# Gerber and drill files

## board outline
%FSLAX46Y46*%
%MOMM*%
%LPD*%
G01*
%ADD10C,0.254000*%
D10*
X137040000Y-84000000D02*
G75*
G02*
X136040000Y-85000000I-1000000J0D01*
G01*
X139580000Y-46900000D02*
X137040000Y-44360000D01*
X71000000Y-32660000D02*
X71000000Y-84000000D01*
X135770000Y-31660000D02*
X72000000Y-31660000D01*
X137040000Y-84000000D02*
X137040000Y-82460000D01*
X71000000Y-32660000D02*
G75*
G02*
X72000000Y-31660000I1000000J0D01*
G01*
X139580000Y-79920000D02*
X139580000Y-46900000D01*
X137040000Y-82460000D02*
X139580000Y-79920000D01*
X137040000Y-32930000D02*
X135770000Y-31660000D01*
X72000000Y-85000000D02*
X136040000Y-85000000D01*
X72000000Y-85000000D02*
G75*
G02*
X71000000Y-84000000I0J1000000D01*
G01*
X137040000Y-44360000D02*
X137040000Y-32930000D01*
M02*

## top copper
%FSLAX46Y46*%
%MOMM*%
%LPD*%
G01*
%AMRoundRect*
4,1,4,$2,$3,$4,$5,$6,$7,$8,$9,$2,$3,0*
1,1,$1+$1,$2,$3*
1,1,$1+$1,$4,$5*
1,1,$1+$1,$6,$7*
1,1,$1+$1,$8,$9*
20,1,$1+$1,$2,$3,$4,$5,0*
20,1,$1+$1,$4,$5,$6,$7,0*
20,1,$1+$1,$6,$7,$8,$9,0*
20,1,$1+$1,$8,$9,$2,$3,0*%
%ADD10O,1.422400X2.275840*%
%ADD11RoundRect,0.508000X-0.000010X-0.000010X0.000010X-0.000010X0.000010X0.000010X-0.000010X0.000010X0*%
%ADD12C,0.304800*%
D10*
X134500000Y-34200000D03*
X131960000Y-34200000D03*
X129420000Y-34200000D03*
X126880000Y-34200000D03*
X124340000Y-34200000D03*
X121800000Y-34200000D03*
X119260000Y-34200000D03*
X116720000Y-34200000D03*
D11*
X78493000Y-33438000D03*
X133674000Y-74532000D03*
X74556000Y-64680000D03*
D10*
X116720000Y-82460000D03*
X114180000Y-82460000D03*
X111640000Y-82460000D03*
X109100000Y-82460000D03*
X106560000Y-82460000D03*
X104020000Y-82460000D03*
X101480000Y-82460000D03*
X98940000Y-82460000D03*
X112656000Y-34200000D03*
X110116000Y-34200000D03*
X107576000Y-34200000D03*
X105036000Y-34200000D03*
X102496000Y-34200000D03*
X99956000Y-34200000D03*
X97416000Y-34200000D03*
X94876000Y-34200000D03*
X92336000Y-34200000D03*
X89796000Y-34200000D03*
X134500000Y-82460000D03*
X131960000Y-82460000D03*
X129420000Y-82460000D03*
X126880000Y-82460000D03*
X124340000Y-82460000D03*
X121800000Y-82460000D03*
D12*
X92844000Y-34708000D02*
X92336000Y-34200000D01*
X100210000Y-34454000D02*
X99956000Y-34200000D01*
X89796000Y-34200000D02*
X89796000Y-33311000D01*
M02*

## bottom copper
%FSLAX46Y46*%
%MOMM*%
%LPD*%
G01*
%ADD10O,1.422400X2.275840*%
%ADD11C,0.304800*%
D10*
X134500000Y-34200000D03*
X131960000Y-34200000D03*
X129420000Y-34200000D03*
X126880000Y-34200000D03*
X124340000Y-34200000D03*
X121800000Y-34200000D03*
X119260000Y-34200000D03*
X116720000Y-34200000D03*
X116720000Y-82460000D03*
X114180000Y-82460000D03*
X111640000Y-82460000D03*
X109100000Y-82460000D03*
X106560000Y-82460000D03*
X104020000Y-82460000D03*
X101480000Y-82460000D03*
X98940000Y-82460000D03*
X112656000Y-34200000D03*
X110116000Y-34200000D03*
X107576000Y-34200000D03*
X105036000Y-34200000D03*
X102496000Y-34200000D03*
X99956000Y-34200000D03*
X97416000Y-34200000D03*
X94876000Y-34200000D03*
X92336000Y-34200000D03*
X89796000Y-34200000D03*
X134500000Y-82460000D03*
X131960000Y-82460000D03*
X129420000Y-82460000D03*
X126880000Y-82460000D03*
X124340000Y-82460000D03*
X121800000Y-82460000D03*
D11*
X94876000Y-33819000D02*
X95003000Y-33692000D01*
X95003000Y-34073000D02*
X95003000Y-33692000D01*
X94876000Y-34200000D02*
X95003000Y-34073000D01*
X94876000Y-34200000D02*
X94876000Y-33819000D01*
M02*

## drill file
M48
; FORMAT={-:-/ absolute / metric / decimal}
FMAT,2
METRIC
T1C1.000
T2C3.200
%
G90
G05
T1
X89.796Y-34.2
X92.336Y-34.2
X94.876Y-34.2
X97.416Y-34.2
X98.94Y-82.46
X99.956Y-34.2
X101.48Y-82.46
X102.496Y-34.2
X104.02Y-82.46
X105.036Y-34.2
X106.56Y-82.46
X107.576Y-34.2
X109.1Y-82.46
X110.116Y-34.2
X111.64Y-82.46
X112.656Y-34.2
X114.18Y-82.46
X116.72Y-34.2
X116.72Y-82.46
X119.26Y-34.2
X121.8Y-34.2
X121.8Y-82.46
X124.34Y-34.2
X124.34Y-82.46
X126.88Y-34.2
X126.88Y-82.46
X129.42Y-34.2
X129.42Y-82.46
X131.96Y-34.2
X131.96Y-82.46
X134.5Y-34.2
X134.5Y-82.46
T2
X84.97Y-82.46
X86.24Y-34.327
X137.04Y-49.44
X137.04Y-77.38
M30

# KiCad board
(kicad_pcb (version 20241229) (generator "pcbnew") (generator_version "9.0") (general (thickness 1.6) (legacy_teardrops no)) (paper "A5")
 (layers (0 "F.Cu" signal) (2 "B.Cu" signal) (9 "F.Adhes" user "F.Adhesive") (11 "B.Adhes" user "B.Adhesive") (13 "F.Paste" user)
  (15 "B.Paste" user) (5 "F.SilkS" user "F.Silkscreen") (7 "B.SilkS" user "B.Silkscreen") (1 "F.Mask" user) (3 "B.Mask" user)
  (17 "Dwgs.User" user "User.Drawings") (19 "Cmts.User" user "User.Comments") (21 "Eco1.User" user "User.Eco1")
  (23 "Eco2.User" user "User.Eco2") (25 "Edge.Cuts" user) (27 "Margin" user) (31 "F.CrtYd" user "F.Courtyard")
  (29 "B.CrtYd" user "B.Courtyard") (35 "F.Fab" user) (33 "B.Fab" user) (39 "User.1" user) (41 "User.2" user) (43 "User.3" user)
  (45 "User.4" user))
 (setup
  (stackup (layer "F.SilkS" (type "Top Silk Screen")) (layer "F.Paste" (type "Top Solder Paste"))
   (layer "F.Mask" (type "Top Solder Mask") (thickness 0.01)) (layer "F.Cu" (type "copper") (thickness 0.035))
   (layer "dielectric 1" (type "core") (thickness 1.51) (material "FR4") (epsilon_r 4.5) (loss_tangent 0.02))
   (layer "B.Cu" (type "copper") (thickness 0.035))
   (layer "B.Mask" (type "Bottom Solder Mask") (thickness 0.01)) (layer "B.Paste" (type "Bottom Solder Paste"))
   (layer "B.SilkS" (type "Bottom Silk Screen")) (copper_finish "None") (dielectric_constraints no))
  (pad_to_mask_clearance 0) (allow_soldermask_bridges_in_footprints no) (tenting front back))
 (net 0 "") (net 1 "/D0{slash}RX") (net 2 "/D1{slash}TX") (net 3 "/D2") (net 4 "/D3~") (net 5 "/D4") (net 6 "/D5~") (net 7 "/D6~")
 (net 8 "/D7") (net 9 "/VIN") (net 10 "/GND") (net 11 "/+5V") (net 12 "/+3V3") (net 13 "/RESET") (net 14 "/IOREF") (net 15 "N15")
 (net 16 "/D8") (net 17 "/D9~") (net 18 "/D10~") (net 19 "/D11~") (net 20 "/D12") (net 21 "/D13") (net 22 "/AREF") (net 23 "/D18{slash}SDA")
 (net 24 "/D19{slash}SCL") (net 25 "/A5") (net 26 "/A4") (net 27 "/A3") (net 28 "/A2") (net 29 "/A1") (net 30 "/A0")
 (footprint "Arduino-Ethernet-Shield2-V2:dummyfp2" (layer "F.Cu") (at 86.24 34.327)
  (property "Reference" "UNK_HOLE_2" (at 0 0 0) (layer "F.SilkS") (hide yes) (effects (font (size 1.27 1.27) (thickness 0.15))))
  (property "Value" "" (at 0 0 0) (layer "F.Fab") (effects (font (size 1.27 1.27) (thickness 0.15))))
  (pad "" np_thru_hole circle (at 0 0) (size 3.2 3.2) (drill 3.2) (layers "*.Cu" "*.Mask")))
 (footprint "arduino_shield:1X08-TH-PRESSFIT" (layer "F.Cu") (at 125.61 34.2 180)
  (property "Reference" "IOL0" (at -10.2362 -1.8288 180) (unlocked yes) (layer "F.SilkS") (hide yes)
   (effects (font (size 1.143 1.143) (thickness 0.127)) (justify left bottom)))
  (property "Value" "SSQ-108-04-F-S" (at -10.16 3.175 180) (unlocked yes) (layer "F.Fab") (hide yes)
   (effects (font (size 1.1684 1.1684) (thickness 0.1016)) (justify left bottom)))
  (pad "1" thru_hole oval (at -8.89 0 270) (size 2.27584 1.4224) (drill 1) (layers "*.Cu" "*.Mask") (remove_unused_layers no)
   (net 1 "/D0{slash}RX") (solder_mask_margin 0.0508) (thermal_bridge_angle 0))
  (pad "2" thru_hole oval (at -6.35 0 270) (size 2.27584 1.4224) (drill 1) (layers "*.Cu" "*.Mask") (remove_unused_layers no)
   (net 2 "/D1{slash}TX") (solder_mask_margin 0.0508) (thermal_bridge_angle 0))
  (pad "3" thru_hole oval (at -3.81 0 270) (size 2.27584 1.4224) (drill 1) (layers "*.Cu" "*.Mask") (remove_unused_layers no) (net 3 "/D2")
   (solder_mask_margin 0.0508) (thermal_bridge_angle 0))
  (pad "4" thru_hole oval (at -1.27 0 270) (size 2.27584 1.4224) (drill 1) (layers "*.Cu" "*.Mask") (remove_unused_layers no) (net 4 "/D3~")
   (solder_mask_margin 0.0508) (thermal_bridge_angle 0))
  (pad "5" thru_hole oval (at 1.27 0 270) (size 2.27584 1.4224) (drill 1) (layers "*.Cu" "*.Mask") (remove_unused_layers no) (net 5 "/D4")
   (solder_mask_margin 0.0508) (thermal_bridge_angle 0))
  (pad "6" thru_hole oval (at 3.81 0 270) (size 2.27584 1.4224) (drill 1) (layers "*.Cu" "*.Mask") (remove_unused_layers no) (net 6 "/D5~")
   (solder_mask_margin 0.0508) (thermal_bridge_angle 0))
  (pad "7" thru_hole oval (at 6.35 0 270) (size 2.27584 1.4224) (drill 1) (layers "*.Cu" "*.Mask") (remove_unused_layers no) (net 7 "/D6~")
   (solder_mask_margin 0.0508) (thermal_bridge_angle 0))
  (pad "8" thru_hole oval (at 8.89 0 270) (size 2.27584 1.4224) (drill 1) (layers "*.Cu" "*.Mask") (remove_unused_layers no) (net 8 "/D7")
   (solder_mask_margin 0.0508) (thermal_bridge_angle 0)))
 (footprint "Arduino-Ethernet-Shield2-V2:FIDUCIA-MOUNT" (layer "F.Cu") (at 78.493 33.438)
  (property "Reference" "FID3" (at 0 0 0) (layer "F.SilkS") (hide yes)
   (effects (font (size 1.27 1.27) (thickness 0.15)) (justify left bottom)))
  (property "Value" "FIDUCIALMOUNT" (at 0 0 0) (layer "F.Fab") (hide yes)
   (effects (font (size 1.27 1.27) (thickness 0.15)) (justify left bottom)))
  (pad "P$1" smd roundrect (at 0 0) (size 1.016 1.016) (layers "F.Cu" "F.Mask" "F.Paste") (roundrect_rratio 0.5) (solder_mask_margin 0.0508)
   (solder_paste_margin -0.0508) (thermal_bridge_angle 0))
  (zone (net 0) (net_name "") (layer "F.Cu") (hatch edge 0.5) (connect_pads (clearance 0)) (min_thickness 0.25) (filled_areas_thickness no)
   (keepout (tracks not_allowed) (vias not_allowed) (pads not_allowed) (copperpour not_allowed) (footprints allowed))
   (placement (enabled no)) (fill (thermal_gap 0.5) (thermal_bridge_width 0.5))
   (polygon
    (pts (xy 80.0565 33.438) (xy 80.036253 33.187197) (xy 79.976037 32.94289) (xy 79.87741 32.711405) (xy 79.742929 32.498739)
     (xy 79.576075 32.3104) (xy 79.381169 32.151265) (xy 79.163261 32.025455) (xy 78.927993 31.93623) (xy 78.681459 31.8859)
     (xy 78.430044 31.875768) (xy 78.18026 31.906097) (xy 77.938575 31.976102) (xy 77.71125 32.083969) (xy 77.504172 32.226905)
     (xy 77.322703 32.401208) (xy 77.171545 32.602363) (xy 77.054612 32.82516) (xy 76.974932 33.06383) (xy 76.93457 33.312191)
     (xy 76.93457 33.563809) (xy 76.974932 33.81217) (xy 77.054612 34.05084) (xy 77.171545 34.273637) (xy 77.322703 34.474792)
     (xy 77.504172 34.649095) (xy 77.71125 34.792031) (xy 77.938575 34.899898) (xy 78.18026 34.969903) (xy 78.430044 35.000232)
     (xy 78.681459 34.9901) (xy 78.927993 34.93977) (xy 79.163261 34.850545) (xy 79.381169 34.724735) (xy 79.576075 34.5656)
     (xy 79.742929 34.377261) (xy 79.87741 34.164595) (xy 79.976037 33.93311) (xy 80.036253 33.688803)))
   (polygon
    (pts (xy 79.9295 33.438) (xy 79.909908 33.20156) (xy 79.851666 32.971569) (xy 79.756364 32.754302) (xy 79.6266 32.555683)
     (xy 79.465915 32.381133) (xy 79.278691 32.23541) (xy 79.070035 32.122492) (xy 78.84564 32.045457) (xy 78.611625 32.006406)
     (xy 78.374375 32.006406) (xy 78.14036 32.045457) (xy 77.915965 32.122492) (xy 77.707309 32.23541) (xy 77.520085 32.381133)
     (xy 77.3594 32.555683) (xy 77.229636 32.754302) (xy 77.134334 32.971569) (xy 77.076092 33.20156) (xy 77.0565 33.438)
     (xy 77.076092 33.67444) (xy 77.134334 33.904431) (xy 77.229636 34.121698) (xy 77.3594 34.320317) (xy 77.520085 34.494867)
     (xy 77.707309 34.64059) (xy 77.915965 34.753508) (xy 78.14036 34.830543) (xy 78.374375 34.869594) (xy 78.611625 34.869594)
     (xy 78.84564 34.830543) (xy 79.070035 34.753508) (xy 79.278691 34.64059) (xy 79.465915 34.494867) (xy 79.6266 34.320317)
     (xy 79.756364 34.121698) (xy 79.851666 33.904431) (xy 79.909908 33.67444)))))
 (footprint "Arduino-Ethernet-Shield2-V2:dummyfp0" (layer "F.Cu") (at 137.04 49.44)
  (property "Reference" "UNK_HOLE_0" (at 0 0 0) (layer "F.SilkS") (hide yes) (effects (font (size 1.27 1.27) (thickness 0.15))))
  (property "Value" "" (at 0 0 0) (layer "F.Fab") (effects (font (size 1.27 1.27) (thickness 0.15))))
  (pad "" np_thru_hole circle (at 0 0) (size 3.2 3.2) (drill 3.2) (layers "*.Cu" "*.Mask")))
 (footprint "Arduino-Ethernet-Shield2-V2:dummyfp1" (layer "F.Cu") (at 137.04 77.38)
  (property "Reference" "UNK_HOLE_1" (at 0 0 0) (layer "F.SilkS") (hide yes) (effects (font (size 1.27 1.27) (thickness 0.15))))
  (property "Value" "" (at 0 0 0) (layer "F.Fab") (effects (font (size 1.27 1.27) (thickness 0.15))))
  (pad "" np_thru_hole circle (at 0 0) (size 3.2 3.2) (drill 3.2) (layers "*.Cu" "*.Mask")))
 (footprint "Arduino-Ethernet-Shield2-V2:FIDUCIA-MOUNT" (layer "F.Cu") (at 133.674 74.532)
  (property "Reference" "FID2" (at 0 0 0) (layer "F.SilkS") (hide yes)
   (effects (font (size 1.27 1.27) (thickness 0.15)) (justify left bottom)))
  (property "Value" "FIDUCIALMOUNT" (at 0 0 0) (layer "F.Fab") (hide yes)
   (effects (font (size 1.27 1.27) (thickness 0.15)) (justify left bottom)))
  (pad "P$1" smd roundrect (at 0 0) (size 1.016 1.016) (layers "F.Cu" "F.Mask" "F.Paste") (roundrect_rratio 0.5) (solder_mask_margin 0.0508)
   (solder_paste_margin -0.0508) (thermal_bridge_angle 0))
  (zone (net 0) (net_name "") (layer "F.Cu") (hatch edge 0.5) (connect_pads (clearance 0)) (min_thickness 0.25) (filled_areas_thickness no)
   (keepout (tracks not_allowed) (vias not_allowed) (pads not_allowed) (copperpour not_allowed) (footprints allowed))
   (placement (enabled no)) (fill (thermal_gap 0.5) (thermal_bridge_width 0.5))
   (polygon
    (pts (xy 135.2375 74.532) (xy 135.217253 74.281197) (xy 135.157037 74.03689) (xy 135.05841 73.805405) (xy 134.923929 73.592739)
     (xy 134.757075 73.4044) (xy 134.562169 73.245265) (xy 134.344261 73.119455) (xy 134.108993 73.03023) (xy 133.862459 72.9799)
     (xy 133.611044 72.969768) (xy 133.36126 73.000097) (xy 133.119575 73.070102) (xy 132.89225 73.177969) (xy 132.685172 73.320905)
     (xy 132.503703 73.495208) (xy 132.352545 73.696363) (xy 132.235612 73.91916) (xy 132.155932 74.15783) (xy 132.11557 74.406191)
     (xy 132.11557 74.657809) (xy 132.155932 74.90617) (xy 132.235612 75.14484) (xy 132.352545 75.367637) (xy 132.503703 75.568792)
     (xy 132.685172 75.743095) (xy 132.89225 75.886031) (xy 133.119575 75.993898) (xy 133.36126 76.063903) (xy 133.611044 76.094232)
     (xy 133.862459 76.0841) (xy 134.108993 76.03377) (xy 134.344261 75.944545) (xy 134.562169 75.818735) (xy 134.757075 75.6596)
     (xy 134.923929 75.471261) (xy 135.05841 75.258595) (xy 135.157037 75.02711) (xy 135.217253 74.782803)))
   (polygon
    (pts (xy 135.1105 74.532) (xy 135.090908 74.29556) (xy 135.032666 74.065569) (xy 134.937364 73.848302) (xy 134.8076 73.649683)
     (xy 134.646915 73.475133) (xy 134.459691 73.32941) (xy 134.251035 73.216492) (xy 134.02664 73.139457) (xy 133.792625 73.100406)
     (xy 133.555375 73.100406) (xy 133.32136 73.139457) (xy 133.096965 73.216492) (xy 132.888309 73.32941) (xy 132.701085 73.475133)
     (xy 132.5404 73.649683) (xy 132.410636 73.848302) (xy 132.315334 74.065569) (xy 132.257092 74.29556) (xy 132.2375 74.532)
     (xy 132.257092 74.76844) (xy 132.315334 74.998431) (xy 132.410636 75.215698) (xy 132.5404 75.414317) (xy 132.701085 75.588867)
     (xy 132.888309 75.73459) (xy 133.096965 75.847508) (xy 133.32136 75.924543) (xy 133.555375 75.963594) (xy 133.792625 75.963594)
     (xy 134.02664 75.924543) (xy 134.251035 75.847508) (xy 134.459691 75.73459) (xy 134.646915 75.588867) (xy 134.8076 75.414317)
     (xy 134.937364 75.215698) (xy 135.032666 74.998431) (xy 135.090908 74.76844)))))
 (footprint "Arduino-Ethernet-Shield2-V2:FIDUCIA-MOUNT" (layer "F.Cu") (at 74.556 64.68)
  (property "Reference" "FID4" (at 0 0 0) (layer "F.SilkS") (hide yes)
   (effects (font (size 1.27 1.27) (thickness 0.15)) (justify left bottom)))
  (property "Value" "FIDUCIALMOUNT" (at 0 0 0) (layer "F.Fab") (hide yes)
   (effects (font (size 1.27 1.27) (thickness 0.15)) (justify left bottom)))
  (pad "P$1" smd roundrect (at 0 0) (size 1.016 1.016) (layers "F.Cu" "F.Mask" "F.Paste") (roundrect_rratio 0.5) (solder_mask_margin 0.0508)
   (solder_paste_margin -0.0508) (thermal_bridge_angle 0))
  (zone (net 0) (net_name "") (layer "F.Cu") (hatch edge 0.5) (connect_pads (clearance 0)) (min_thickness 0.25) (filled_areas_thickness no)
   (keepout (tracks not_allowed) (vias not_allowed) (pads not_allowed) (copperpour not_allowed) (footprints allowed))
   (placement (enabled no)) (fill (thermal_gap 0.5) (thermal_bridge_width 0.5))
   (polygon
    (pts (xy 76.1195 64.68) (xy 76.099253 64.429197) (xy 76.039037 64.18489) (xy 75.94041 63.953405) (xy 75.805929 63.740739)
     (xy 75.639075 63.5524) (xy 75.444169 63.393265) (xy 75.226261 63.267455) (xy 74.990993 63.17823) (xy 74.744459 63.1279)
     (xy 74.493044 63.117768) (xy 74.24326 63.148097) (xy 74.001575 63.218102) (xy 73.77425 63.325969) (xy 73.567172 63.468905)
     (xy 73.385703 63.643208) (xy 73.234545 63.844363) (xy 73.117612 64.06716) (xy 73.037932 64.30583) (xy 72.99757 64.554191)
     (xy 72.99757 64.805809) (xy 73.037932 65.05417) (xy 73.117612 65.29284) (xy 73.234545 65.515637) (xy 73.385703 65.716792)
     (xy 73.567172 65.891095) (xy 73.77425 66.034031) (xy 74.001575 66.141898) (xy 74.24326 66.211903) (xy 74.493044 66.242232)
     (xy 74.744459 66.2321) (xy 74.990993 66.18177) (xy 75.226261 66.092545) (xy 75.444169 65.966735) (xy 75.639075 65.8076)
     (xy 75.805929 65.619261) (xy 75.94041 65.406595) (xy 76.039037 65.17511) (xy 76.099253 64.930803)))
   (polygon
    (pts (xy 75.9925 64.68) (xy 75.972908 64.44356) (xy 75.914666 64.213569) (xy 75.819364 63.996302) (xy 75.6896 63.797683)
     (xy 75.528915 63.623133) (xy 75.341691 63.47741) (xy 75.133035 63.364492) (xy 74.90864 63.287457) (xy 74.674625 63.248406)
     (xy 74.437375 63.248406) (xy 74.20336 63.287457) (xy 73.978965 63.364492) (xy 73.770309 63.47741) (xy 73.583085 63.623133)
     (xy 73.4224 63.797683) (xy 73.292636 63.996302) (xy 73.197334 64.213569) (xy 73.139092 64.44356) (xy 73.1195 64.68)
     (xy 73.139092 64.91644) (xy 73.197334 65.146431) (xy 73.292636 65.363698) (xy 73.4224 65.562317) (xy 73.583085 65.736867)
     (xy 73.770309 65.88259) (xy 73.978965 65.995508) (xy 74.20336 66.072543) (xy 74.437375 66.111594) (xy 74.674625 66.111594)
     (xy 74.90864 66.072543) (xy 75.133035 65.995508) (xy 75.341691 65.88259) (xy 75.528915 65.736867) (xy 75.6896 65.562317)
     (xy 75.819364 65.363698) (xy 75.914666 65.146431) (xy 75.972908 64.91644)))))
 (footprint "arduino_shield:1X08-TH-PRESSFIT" (layer "F.Cu") (at 107.83 82.46 180)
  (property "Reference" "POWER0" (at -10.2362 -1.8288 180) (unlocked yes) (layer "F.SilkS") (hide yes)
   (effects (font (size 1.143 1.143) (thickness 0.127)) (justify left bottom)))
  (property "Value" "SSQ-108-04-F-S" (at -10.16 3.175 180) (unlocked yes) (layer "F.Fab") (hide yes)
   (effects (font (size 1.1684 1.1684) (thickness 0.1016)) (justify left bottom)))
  (pad "1" thru_hole oval (at -8.89 0 270) (size 2.27584 1.4224) (drill 1) (layers "*.Cu" "*.Mask") (remove_unused_layers no) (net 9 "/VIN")
   (solder_mask_margin 0.0508) (thermal_bridge_angle 0))
  (pad "2" thru_hole oval (at -6.35 0 270) (size 2.27584 1.4224) (drill 1) (layers "*.Cu" "*.Mask") (remove_unused_layers no)
   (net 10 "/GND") (solder_mask_margin 0.0508) (thermal_bridge_angle 0))
  (pad "3" thru_hole oval (at -3.81 0 270) (size 2.27584 1.4224) (drill 1) (layers "*.Cu" "*.Mask") (remove_unused_layers no)
   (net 10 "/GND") (solder_mask_margin 0.0508) (thermal_bridge_angle 0))
  (pad "4" thru_hole oval (at -1.27 0 270) (size 2.27584 1.4224) (drill 1) (layers "*.Cu" "*.Mask") (remove_unused_layers no)
   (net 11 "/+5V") (solder_mask_margin 0.0508) (thermal_bridge_angle 0))
  (pad "5" thru_hole oval (at 1.27 0 270) (size 2.27584 1.4224) (drill 1) (layers "*.Cu" "*.Mask") (remove_unused_layers no)
   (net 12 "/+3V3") (solder_mask_margin 0.0508) (thermal_bridge_angle 0))
  (pad "6" thru_hole oval (at 3.81 0 270) (size 2.27584 1.4224) (drill 1) (layers "*.Cu" "*.Mask") (remove_unused_layers no)
   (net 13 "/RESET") (solder_mask_margin 0.0508) (thermal_bridge_angle 0))
  (pad "7" thru_hole oval (at 6.35 0 270) (size 2.27584 1.4224) (drill 1) (layers "*.Cu" "*.Mask") (remove_unused_layers no)
   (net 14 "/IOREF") (solder_mask_margin 0.0508) (thermal_bridge_angle 0))
  (pad "8" thru_hole oval (at 8.89 0 270) (size 2.27584 1.4224) (drill 1) (layers "*.Cu" "*.Mask") (remove_unused_layers no) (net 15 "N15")
   (solder_mask_margin 0.0508) (thermal_bridge_angle 0)))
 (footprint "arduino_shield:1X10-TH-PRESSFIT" (layer "F.Cu") (at 101.226 34.2 180)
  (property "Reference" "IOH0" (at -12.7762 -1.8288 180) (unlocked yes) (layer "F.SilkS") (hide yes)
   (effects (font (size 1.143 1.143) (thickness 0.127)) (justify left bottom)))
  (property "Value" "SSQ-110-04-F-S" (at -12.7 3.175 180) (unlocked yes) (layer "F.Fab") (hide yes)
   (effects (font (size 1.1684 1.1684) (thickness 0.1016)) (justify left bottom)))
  (pad "1" thru_hole oval (at -11.43 0 270) (size 2.27584 1.4224) (drill 1) (layers "*.Cu" "*.Mask") (remove_unused_layers no)
   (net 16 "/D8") (solder_mask_margin 0.0508) (thermal_bridge_angle 0))
  (pad "2" thru_hole oval (at -8.89 0 270) (size 2.27584 1.4224) (drill 1) (layers "*.Cu" "*.Mask") (remove_unused_layers no)
   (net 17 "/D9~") (solder_mask_margin 0.0508) (thermal_bridge_angle 0))
  (pad "3" thru_hole oval (at -6.35 0 270) (size 2.27584 1.4224) (drill 1) (layers "*.Cu" "*.Mask") (remove_unused_layers no)
   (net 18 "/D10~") (solder_mask_margin 0.0508) (thermal_bridge_angle 0))
  (pad "4" thru_hole oval (at -3.81 0 270) (size 2.27584 1.4224) (drill 1) (layers "*.Cu" "*.Mask") (remove_unused_layers no)
   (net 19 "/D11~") (solder_mask_margin 0.0508) (thermal_bridge_angle 0))
  (pad "5" thru_hole oval (at -1.27 0 270) (size 2.27584 1.4224) (drill 1) (layers "*.Cu" "*.Mask") (remove_unused_layers no)
   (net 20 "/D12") (solder_mask_margin 0.0508) (thermal_bridge_angle 0))
  (pad "6" thru_hole oval (at 1.27 0 270) (size 2.27584 1.4224) (drill 1) (layers "*.Cu" "*.Mask") (remove_unused_layers no) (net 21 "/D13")
   (solder_mask_margin 0.0508) (thermal_bridge_angle 0))
  (pad "7" thru_hole oval (at 3.81 0 270) (size 2.27584 1.4224) (drill 1) (layers "*.Cu" "*.Mask") (remove_unused_layers no) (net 10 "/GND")
   (solder_mask_margin 0.0508) (thermal_bridge_angle 0))
  (pad "8" thru_hole oval (at 6.35 0 270) (size 2.27584 1.4224) (drill 1) (layers "*.Cu" "*.Mask") (remove_unused_layers no)
   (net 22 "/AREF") (solder_mask_margin 0.0508) (thermal_bridge_angle 0))
  (pad "9" thru_hole oval (at 8.89 0 270) (size 2.27584 1.4224) (drill 1) (layers "*.Cu" "*.Mask") (remove_unused_layers no)
   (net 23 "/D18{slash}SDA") (solder_mask_margin 0.0508) (thermal_bridge_angle 0))
  (pad "10" thru_hole oval (at 11.43 0 270) (size 2.27584 1.4224) (drill 1) (layers "*.Cu" "*.Mask") (remove_unused_layers no)
   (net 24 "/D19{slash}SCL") (solder_mask_margin 0.0508) (thermal_bridge_angle 0)))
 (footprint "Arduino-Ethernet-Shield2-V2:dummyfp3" (layer "F.Cu") (at 84.97 82.46)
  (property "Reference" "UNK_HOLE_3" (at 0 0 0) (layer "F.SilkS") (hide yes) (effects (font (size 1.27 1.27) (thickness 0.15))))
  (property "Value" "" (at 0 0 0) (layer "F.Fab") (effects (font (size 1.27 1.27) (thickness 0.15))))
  (pad "" np_thru_hole circle (at 0 0) (size 3.2 3.2) (drill 3.2) (layers "*.Cu" "*.Mask")))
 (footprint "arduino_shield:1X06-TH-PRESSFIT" (layer "F.Cu") (at 128.15 82.46 180)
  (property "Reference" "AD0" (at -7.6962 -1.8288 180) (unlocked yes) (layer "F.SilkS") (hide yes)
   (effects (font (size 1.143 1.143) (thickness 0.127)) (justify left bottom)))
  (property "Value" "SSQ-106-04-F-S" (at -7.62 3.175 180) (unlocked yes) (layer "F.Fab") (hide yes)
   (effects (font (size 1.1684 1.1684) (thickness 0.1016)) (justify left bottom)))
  (pad "1" thru_hole oval (at -6.35 0 270) (size 2.27584 1.4224) (drill 1) (layers "*.Cu" "*.Mask") (remove_unused_layers no) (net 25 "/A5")
   (solder_mask_margin 0.0508) (thermal_bridge_angle 0))
  (pad "2" thru_hole oval (at -3.81 0 270) (size 2.27584 1.4224) (drill 1) (layers "*.Cu" "*.Mask") (remove_unused_layers no) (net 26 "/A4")
   (solder_mask_margin 0.0508) (thermal_bridge_angle 0))
  (pad "3" thru_hole oval (at -1.27 0 270) (size 2.27584 1.4224) (drill 1) (layers "*.Cu" "*.Mask") (remove_unused_layers no) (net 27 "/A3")
   (solder_mask_margin 0.0508) (thermal_bridge_angle 0))
  (pad "4" thru_hole oval (at 1.27 0 270) (size 2.27584 1.4224) (drill 1) (layers "*.Cu" "*.Mask") (remove_unused_layers no) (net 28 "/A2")
   (solder_mask_margin 0.0508) (thermal_bridge_angle 0))
  (pad "5" thru_hole oval (at 3.81 0 270) (size 2.27584 1.4224) (drill 1) (layers "*.Cu" "*.Mask") (remove_unused_layers no) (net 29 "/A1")
   (solder_mask_margin 0.0508) (thermal_bridge_angle 0))
  (pad "6" thru_hole oval (at 6.35 0 270) (size 2.27584 1.4224) (drill 1) (layers "*.Cu" "*.Mask") (remove_unused_layers no) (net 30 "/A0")
   (solder_mask_margin 0.0508) (thermal_bridge_angle 0)))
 (gr_arc (start 137.04 84) (mid 136.747107 84.707107) (end 136.04 85) (stroke (width 0.254) (type solid)) (layer "Edge.Cuts"))
 (gr_line (start 139.58 46.9) (end 137.04 44.36) (stroke (width 0.254) (type solid)) (layer "Edge.Cuts"))
 (gr_line (start 71 32.66) (end 71 84) (stroke (width 0.254) (type solid)) (layer "Edge.Cuts"))
 (gr_line (start 135.77 31.66) (end 72 31.66) (stroke (width 0.254) (type solid)) (layer "Edge.Cuts"))
 (gr_line (start 137.04 84) (end 137.04 82.46) (stroke (width 0.254) (type solid)) (layer "Edge.Cuts"))
 (gr_arc (start 71 32.66) (mid 71.292893 31.952893) (end 72 31.66) (stroke (width 0.254) (type solid)) (layer "Edge.Cuts"))
 (gr_line (start 139.58 79.92) (end 139.58 46.9) (stroke (width 0.254) (type solid)) (layer "Edge.Cuts"))
 (gr_line (start 137.04 82.46) (end 139.58 79.92) (stroke (width 0.254) (type solid)) (layer "Edge.Cuts"))
 (gr_line (start 137.04 32.93) (end 135.77 31.66) (stroke (width 0.254) (type solid)) (layer "Edge.Cuts"))
 (gr_line (start 72 85) (end 136.04 85) (stroke (width 0.254) (type solid)) (layer "Edge.Cuts"))
 (gr_arc (start 72 85) (mid 71.292893 84.707107) (end 71 84) (stroke (width 0.254) (type solid)) (layer "Edge.Cuts"))
 (gr_line (start 137.04 44.36) (end 137.04 32.93) (stroke (width 0.254) (type solid)) (layer "Edge.Cuts"))
 (segment (start 92.844 34.708) (end 92.336 34.2) (width 0.3048) (layer "F.Cu") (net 23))
 (segment (start 100.21 34.454) (end 99.956 34.2) (width 0.3048) (layer "F.Cu") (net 21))
 (segment (start 89.796 34.2) (end 89.796 33.311) (width 0.3048) (layer "F.Cu") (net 24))
 (segment (start 94.876 33.819) (end 95.003 33.692) (width 0.3048) (layer "B.Cu") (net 22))
 (segment (start 95.003 34.073) (end 95.003 33.692) (width 0.3048) (layer "B.Cu") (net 22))
 (segment (start 94.876 34.2) (end 95.003 34.073) (width 0.3048) (layer "B.Cu") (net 22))
 (segment (start 94.876 34.2) (end 94.876 33.819) (width 0.3048) (layer "B.Cu") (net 22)))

